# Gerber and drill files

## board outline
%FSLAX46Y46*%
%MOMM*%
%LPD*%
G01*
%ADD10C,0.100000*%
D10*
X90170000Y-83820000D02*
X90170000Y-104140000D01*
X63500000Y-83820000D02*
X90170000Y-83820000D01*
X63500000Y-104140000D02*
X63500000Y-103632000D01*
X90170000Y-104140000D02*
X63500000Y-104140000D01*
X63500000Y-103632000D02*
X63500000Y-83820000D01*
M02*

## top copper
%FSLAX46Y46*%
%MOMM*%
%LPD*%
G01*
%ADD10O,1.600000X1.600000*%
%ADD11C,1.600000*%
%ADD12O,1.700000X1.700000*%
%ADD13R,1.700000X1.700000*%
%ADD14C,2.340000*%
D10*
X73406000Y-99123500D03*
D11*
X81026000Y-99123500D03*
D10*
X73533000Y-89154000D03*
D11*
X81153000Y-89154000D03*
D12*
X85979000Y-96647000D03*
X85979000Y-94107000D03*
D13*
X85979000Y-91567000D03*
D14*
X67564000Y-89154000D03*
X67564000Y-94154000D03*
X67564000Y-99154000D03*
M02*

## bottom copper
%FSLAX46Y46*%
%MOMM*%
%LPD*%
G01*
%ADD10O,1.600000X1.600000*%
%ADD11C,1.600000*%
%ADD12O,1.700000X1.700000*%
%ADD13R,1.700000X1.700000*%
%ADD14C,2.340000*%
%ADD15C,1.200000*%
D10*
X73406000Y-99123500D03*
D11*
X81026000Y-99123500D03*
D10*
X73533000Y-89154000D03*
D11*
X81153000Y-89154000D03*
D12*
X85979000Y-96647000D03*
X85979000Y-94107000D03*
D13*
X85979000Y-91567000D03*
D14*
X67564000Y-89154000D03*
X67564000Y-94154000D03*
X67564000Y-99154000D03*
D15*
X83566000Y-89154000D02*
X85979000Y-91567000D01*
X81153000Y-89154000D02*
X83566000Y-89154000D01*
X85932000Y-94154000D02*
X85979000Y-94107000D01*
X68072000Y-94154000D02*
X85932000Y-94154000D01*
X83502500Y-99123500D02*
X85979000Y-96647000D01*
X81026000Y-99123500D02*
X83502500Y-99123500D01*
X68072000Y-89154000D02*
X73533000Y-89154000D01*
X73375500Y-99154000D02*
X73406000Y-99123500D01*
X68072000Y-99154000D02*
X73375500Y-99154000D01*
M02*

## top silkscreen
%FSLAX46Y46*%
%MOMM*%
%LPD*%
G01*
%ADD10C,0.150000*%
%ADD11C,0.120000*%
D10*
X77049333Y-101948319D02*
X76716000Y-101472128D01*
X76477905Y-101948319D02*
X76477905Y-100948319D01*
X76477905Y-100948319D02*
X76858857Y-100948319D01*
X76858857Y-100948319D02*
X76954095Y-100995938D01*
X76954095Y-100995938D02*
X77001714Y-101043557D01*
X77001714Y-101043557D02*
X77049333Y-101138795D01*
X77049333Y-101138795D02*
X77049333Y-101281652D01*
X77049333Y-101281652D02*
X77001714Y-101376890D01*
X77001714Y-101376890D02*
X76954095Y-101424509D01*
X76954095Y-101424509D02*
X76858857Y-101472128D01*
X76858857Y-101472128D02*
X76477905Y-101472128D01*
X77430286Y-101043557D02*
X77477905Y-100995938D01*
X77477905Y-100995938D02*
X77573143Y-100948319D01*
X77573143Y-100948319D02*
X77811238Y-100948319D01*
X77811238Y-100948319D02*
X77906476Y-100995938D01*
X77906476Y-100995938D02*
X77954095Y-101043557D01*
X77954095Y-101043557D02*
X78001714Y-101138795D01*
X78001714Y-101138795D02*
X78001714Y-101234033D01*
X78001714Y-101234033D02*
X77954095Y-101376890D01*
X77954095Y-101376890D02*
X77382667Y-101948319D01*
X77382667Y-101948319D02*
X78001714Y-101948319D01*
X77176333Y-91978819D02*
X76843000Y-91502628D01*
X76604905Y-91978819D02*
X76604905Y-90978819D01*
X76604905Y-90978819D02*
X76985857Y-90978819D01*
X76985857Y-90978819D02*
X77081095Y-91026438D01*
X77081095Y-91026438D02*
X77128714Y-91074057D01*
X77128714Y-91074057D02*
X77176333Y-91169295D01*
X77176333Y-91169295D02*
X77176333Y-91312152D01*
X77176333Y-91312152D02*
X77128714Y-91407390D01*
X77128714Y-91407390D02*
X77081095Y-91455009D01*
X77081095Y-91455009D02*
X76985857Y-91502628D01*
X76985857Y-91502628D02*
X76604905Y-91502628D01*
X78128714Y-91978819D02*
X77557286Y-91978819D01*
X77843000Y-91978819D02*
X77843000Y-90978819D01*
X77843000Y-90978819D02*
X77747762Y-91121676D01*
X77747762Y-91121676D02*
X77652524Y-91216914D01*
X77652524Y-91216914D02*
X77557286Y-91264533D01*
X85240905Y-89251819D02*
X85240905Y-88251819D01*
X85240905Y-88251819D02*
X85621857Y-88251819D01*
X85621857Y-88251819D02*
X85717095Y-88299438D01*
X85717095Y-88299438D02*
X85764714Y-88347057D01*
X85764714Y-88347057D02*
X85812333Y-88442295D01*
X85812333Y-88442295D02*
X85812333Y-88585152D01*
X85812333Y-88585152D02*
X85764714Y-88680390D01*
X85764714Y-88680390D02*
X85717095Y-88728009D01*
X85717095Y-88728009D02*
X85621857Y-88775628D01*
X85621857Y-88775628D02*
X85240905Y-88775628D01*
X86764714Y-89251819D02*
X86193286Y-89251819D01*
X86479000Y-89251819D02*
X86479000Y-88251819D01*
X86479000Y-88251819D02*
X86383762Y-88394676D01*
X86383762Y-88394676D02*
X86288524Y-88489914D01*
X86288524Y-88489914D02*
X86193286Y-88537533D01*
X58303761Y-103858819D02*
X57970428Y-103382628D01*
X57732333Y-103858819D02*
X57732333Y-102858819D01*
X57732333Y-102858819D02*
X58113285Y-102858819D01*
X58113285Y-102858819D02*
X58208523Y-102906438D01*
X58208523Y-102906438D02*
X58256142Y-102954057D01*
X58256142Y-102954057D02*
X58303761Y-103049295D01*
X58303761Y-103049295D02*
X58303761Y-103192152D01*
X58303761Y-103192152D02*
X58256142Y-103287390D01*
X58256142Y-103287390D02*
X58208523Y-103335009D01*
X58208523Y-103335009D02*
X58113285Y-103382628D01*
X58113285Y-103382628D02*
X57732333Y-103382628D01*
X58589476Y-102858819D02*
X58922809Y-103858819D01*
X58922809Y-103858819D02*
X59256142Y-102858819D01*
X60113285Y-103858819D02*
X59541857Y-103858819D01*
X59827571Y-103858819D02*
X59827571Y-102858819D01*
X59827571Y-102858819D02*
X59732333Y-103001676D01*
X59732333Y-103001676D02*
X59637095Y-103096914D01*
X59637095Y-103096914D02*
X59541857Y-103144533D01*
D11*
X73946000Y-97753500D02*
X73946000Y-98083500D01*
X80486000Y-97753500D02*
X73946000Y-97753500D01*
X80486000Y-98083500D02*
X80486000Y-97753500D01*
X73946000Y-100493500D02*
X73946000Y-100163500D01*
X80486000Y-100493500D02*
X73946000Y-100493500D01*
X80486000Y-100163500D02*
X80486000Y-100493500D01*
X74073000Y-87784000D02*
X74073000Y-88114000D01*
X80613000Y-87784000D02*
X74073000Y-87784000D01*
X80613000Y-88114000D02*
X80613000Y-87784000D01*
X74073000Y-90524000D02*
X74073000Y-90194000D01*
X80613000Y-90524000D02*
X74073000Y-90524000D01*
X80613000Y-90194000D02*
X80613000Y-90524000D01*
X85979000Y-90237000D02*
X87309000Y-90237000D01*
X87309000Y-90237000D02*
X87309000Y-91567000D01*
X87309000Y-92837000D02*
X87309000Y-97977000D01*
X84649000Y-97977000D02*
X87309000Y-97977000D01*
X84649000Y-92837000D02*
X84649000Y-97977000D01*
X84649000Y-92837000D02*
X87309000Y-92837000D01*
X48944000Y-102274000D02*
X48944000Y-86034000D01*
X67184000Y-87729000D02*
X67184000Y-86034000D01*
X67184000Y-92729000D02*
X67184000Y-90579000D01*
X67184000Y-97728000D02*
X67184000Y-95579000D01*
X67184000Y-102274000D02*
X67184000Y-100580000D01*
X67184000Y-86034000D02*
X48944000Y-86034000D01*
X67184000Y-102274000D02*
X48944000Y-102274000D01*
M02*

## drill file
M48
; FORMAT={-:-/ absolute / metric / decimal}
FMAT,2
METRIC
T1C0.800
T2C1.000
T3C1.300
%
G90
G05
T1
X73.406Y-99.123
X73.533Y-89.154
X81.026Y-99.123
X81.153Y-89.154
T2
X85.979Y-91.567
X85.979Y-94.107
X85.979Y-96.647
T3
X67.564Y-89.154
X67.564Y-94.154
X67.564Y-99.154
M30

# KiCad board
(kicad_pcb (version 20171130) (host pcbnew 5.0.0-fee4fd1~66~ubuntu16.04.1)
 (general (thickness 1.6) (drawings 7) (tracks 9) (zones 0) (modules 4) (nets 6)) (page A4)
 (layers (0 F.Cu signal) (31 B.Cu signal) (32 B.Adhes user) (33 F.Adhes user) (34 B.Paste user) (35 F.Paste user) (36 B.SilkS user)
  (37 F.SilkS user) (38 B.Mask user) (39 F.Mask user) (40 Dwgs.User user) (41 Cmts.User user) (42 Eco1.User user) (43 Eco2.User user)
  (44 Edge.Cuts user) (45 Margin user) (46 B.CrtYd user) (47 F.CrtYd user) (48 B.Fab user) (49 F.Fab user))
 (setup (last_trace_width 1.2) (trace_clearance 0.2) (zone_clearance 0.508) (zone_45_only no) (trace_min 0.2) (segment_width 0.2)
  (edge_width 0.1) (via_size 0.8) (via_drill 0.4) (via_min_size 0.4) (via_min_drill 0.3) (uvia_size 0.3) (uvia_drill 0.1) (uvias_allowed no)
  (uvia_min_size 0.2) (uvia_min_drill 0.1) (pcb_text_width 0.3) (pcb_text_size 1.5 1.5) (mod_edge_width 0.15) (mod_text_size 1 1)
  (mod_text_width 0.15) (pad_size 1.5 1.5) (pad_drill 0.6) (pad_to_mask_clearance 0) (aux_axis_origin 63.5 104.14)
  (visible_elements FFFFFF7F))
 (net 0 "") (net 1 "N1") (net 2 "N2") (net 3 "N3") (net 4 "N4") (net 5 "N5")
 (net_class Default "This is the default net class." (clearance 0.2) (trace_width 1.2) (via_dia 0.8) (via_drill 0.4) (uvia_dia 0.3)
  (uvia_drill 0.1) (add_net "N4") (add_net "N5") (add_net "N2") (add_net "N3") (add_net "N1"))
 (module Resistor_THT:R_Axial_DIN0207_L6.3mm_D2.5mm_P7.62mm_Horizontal (layer F.Cu) (at 81.026 99.1235 180)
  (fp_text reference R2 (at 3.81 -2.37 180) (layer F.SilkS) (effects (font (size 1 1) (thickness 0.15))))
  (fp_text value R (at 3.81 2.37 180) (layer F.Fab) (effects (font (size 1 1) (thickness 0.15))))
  (fp_line (start 7.08 1.37) (end 7.08 1.04) (layer F.SilkS) (width 0.12))
  (fp_line (start 0.54 1.37) (end 7.08 1.37) (layer F.SilkS) (width 0.12))
  (fp_line (start 0.54 1.04) (end 0.54 1.37) (layer F.SilkS) (width 0.12))
  (fp_line (start 7.08 -1.37) (end 7.08 -1.04) (layer F.SilkS) (width 0.12))
  (fp_line (start 0.54 -1.37) (end 7.08 -1.37) (layer F.SilkS) (width 0.12))
  (fp_line (start 0.54 -1.04) (end 0.54 -1.37) (layer F.SilkS) (width 0.12))
  (pad 2 thru_hole oval (at 7.62 0 180) (size 1.6 1.6) (drill 0.8) (layers *.Cu *.Mask) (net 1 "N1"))
  (pad 1 thru_hole circle (at 0 0 180) (size 1.6 1.6) (drill 0.8) (layers *.Cu *.Mask) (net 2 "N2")))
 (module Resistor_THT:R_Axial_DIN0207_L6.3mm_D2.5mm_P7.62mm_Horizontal (layer F.Cu) (at 81.153 89.154 180)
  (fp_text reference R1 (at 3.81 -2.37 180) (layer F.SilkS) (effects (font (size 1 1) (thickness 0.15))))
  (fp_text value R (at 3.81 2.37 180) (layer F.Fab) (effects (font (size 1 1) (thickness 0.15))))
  (fp_line (start 7.08 1.37) (end 7.08 1.04) (layer F.SilkS) (width 0.12))
  (fp_line (start 0.54 1.37) (end 7.08 1.37) (layer F.SilkS) (width 0.12))
  (fp_line (start 0.54 1.04) (end 0.54 1.37) (layer F.SilkS) (width 0.12))
  (fp_line (start 7.08 -1.37) (end 7.08 -1.04) (layer F.SilkS) (width 0.12))
  (fp_line (start 0.54 -1.37) (end 7.08 -1.37) (layer F.SilkS) (width 0.12))
  (fp_line (start 0.54 -1.04) (end 0.54 -1.37) (layer F.SilkS) (width 0.12))
  (pad 2 thru_hole oval (at 7.62 0 180) (size 1.6 1.6) (drill 0.8) (layers *.Cu *.Mask) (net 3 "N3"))
  (pad 1 thru_hole circle (at 0 0 180) (size 1.6 1.6) (drill 0.8) (layers *.Cu *.Mask) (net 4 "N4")))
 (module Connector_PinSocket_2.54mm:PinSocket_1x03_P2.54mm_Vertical (layer F.Cu) (at 85.979 91.567)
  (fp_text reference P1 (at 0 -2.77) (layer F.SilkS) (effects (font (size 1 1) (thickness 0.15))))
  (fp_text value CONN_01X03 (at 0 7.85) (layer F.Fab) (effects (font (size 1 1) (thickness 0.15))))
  (fp_line (start 0 -1.33) (end 1.33 -1.33) (layer F.SilkS) (width 0.12))
  (fp_line (start 1.33 -1.33) (end 1.33 0) (layer F.SilkS) (width 0.12))
  (fp_line (start 1.33 1.27) (end 1.33 6.41) (layer F.SilkS) (width 0.12))
  (fp_line (start -1.33 6.41) (end 1.33 6.41) (layer F.SilkS) (width 0.12))
  (fp_line (start -1.33 1.27) (end -1.33 6.41) (layer F.SilkS) (width 0.12))
  (fp_line (start -1.33 1.27) (end 1.33 1.27) (layer F.SilkS) (width 0.12))
  (pad 3 thru_hole oval (at 0 5.08) (size 1.7 1.7) (drill 1) (layers *.Cu *.Mask) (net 2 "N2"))
  (pad 2 thru_hole oval (at 0 2.54) (size 1.7 1.7) (drill 1) (layers *.Cu *.Mask) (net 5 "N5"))
  (pad 1 thru_hole rect (at 0 0) (size 1.7 1.7) (drill 1) (layers *.Cu *.Mask) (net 4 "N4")))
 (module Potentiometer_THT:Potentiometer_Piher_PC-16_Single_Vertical (layer F.Cu) (at 67.564 89.154 180)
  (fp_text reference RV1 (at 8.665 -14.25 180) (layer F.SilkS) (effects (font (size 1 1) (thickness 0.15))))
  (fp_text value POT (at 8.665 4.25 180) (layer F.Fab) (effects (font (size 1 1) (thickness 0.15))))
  (fp_line (start 18.62 -13.12) (end 18.62 3.12) (layer F.SilkS) (width 0.12))
  (fp_line (start 0.38 1.425) (end 0.38 3.12) (layer F.SilkS) (width 0.12))
  (fp_line (start 0.38 -3.575) (end 0.38 -1.425) (layer F.SilkS) (width 0.12))
  (fp_line (start 0.38 -8.574) (end 0.38 -6.425) (layer F.SilkS) (width 0.12))
  (fp_line (start 0.38 -13.12) (end 0.38 -11.426) (layer F.SilkS) (width 0.12))
  (fp_line (start 0.38 3.12) (end 18.62 3.12) (layer F.SilkS) (width 0.12))
  (fp_line (start 0.38 -13.12) (end 18.62 -13.12) (layer F.SilkS) (width 0.12))
  (pad 1 thru_hole circle (at 0 0 180) (size 2.34 2.34) (drill 1.3) (layers *.Cu *.Mask) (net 3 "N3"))
  (pad 2 thru_hole circle (at 0 -5 180) (size 2.34 2.34) (drill 1.3) (layers *.Cu *.Mask) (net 5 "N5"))
  (pad 3 thru_hole circle (at 0 -10 180) (size 2.34 2.34) (drill 1.3) (layers *.Cu *.Mask) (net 1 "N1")))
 (gr_line (start 90.17 83.82) (end 90.17 104.14) (layer Edge.Cuts) (width 0.1))
 (gr_line (start 63.5 83.82) (end 90.17 83.82) (layer Edge.Cuts) (width 0.1))
 (gr_line (start 63.5 104.14) (end 63.5 103.632) (layer Edge.Cuts) (width 0.1))
 (gr_line (start 90.17 104.14) (end 63.5 104.14) (layer Edge.Cuts) (width 0.1))
 (gr_line (start 63.5 103.632) (end 63.5 83.82) (layer Edge.Cuts) (width 0.1))
 (segment (start 83.566 89.154) (end 85.979 91.567) (width 1.2) (layer B.Cu) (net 4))
 (segment (start 81.153 89.154) (end 83.566 89.154) (width 1.2) (layer B.Cu) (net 4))
 (segment (start 85.932 94.154) (end 85.979 94.107) (width 1.2) (layer B.Cu) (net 5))
 (segment (start 68.072 94.154) (end 85.932 94.154) (width 1.2) (layer B.Cu) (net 5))
 (segment (start 83.5025 99.1235) (end 85.979 96.647) (width 1.2) (layer B.Cu) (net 2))
 (segment (start 81.026 99.1235) (end 83.5025 99.1235) (width 1.2) (layer B.Cu) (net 2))
 (segment (start 68.072 89.154) (end 73.533 89.154) (width 1.2) (layer B.Cu) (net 3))
 (segment (start 73.3755 99.154) (end 73.406 99.1235) (width 1.2) (layer B.Cu) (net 1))
 (segment (start 68.072 99.154) (end 73.3755 99.154) (width 1.2) (layer B.Cu) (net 1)))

